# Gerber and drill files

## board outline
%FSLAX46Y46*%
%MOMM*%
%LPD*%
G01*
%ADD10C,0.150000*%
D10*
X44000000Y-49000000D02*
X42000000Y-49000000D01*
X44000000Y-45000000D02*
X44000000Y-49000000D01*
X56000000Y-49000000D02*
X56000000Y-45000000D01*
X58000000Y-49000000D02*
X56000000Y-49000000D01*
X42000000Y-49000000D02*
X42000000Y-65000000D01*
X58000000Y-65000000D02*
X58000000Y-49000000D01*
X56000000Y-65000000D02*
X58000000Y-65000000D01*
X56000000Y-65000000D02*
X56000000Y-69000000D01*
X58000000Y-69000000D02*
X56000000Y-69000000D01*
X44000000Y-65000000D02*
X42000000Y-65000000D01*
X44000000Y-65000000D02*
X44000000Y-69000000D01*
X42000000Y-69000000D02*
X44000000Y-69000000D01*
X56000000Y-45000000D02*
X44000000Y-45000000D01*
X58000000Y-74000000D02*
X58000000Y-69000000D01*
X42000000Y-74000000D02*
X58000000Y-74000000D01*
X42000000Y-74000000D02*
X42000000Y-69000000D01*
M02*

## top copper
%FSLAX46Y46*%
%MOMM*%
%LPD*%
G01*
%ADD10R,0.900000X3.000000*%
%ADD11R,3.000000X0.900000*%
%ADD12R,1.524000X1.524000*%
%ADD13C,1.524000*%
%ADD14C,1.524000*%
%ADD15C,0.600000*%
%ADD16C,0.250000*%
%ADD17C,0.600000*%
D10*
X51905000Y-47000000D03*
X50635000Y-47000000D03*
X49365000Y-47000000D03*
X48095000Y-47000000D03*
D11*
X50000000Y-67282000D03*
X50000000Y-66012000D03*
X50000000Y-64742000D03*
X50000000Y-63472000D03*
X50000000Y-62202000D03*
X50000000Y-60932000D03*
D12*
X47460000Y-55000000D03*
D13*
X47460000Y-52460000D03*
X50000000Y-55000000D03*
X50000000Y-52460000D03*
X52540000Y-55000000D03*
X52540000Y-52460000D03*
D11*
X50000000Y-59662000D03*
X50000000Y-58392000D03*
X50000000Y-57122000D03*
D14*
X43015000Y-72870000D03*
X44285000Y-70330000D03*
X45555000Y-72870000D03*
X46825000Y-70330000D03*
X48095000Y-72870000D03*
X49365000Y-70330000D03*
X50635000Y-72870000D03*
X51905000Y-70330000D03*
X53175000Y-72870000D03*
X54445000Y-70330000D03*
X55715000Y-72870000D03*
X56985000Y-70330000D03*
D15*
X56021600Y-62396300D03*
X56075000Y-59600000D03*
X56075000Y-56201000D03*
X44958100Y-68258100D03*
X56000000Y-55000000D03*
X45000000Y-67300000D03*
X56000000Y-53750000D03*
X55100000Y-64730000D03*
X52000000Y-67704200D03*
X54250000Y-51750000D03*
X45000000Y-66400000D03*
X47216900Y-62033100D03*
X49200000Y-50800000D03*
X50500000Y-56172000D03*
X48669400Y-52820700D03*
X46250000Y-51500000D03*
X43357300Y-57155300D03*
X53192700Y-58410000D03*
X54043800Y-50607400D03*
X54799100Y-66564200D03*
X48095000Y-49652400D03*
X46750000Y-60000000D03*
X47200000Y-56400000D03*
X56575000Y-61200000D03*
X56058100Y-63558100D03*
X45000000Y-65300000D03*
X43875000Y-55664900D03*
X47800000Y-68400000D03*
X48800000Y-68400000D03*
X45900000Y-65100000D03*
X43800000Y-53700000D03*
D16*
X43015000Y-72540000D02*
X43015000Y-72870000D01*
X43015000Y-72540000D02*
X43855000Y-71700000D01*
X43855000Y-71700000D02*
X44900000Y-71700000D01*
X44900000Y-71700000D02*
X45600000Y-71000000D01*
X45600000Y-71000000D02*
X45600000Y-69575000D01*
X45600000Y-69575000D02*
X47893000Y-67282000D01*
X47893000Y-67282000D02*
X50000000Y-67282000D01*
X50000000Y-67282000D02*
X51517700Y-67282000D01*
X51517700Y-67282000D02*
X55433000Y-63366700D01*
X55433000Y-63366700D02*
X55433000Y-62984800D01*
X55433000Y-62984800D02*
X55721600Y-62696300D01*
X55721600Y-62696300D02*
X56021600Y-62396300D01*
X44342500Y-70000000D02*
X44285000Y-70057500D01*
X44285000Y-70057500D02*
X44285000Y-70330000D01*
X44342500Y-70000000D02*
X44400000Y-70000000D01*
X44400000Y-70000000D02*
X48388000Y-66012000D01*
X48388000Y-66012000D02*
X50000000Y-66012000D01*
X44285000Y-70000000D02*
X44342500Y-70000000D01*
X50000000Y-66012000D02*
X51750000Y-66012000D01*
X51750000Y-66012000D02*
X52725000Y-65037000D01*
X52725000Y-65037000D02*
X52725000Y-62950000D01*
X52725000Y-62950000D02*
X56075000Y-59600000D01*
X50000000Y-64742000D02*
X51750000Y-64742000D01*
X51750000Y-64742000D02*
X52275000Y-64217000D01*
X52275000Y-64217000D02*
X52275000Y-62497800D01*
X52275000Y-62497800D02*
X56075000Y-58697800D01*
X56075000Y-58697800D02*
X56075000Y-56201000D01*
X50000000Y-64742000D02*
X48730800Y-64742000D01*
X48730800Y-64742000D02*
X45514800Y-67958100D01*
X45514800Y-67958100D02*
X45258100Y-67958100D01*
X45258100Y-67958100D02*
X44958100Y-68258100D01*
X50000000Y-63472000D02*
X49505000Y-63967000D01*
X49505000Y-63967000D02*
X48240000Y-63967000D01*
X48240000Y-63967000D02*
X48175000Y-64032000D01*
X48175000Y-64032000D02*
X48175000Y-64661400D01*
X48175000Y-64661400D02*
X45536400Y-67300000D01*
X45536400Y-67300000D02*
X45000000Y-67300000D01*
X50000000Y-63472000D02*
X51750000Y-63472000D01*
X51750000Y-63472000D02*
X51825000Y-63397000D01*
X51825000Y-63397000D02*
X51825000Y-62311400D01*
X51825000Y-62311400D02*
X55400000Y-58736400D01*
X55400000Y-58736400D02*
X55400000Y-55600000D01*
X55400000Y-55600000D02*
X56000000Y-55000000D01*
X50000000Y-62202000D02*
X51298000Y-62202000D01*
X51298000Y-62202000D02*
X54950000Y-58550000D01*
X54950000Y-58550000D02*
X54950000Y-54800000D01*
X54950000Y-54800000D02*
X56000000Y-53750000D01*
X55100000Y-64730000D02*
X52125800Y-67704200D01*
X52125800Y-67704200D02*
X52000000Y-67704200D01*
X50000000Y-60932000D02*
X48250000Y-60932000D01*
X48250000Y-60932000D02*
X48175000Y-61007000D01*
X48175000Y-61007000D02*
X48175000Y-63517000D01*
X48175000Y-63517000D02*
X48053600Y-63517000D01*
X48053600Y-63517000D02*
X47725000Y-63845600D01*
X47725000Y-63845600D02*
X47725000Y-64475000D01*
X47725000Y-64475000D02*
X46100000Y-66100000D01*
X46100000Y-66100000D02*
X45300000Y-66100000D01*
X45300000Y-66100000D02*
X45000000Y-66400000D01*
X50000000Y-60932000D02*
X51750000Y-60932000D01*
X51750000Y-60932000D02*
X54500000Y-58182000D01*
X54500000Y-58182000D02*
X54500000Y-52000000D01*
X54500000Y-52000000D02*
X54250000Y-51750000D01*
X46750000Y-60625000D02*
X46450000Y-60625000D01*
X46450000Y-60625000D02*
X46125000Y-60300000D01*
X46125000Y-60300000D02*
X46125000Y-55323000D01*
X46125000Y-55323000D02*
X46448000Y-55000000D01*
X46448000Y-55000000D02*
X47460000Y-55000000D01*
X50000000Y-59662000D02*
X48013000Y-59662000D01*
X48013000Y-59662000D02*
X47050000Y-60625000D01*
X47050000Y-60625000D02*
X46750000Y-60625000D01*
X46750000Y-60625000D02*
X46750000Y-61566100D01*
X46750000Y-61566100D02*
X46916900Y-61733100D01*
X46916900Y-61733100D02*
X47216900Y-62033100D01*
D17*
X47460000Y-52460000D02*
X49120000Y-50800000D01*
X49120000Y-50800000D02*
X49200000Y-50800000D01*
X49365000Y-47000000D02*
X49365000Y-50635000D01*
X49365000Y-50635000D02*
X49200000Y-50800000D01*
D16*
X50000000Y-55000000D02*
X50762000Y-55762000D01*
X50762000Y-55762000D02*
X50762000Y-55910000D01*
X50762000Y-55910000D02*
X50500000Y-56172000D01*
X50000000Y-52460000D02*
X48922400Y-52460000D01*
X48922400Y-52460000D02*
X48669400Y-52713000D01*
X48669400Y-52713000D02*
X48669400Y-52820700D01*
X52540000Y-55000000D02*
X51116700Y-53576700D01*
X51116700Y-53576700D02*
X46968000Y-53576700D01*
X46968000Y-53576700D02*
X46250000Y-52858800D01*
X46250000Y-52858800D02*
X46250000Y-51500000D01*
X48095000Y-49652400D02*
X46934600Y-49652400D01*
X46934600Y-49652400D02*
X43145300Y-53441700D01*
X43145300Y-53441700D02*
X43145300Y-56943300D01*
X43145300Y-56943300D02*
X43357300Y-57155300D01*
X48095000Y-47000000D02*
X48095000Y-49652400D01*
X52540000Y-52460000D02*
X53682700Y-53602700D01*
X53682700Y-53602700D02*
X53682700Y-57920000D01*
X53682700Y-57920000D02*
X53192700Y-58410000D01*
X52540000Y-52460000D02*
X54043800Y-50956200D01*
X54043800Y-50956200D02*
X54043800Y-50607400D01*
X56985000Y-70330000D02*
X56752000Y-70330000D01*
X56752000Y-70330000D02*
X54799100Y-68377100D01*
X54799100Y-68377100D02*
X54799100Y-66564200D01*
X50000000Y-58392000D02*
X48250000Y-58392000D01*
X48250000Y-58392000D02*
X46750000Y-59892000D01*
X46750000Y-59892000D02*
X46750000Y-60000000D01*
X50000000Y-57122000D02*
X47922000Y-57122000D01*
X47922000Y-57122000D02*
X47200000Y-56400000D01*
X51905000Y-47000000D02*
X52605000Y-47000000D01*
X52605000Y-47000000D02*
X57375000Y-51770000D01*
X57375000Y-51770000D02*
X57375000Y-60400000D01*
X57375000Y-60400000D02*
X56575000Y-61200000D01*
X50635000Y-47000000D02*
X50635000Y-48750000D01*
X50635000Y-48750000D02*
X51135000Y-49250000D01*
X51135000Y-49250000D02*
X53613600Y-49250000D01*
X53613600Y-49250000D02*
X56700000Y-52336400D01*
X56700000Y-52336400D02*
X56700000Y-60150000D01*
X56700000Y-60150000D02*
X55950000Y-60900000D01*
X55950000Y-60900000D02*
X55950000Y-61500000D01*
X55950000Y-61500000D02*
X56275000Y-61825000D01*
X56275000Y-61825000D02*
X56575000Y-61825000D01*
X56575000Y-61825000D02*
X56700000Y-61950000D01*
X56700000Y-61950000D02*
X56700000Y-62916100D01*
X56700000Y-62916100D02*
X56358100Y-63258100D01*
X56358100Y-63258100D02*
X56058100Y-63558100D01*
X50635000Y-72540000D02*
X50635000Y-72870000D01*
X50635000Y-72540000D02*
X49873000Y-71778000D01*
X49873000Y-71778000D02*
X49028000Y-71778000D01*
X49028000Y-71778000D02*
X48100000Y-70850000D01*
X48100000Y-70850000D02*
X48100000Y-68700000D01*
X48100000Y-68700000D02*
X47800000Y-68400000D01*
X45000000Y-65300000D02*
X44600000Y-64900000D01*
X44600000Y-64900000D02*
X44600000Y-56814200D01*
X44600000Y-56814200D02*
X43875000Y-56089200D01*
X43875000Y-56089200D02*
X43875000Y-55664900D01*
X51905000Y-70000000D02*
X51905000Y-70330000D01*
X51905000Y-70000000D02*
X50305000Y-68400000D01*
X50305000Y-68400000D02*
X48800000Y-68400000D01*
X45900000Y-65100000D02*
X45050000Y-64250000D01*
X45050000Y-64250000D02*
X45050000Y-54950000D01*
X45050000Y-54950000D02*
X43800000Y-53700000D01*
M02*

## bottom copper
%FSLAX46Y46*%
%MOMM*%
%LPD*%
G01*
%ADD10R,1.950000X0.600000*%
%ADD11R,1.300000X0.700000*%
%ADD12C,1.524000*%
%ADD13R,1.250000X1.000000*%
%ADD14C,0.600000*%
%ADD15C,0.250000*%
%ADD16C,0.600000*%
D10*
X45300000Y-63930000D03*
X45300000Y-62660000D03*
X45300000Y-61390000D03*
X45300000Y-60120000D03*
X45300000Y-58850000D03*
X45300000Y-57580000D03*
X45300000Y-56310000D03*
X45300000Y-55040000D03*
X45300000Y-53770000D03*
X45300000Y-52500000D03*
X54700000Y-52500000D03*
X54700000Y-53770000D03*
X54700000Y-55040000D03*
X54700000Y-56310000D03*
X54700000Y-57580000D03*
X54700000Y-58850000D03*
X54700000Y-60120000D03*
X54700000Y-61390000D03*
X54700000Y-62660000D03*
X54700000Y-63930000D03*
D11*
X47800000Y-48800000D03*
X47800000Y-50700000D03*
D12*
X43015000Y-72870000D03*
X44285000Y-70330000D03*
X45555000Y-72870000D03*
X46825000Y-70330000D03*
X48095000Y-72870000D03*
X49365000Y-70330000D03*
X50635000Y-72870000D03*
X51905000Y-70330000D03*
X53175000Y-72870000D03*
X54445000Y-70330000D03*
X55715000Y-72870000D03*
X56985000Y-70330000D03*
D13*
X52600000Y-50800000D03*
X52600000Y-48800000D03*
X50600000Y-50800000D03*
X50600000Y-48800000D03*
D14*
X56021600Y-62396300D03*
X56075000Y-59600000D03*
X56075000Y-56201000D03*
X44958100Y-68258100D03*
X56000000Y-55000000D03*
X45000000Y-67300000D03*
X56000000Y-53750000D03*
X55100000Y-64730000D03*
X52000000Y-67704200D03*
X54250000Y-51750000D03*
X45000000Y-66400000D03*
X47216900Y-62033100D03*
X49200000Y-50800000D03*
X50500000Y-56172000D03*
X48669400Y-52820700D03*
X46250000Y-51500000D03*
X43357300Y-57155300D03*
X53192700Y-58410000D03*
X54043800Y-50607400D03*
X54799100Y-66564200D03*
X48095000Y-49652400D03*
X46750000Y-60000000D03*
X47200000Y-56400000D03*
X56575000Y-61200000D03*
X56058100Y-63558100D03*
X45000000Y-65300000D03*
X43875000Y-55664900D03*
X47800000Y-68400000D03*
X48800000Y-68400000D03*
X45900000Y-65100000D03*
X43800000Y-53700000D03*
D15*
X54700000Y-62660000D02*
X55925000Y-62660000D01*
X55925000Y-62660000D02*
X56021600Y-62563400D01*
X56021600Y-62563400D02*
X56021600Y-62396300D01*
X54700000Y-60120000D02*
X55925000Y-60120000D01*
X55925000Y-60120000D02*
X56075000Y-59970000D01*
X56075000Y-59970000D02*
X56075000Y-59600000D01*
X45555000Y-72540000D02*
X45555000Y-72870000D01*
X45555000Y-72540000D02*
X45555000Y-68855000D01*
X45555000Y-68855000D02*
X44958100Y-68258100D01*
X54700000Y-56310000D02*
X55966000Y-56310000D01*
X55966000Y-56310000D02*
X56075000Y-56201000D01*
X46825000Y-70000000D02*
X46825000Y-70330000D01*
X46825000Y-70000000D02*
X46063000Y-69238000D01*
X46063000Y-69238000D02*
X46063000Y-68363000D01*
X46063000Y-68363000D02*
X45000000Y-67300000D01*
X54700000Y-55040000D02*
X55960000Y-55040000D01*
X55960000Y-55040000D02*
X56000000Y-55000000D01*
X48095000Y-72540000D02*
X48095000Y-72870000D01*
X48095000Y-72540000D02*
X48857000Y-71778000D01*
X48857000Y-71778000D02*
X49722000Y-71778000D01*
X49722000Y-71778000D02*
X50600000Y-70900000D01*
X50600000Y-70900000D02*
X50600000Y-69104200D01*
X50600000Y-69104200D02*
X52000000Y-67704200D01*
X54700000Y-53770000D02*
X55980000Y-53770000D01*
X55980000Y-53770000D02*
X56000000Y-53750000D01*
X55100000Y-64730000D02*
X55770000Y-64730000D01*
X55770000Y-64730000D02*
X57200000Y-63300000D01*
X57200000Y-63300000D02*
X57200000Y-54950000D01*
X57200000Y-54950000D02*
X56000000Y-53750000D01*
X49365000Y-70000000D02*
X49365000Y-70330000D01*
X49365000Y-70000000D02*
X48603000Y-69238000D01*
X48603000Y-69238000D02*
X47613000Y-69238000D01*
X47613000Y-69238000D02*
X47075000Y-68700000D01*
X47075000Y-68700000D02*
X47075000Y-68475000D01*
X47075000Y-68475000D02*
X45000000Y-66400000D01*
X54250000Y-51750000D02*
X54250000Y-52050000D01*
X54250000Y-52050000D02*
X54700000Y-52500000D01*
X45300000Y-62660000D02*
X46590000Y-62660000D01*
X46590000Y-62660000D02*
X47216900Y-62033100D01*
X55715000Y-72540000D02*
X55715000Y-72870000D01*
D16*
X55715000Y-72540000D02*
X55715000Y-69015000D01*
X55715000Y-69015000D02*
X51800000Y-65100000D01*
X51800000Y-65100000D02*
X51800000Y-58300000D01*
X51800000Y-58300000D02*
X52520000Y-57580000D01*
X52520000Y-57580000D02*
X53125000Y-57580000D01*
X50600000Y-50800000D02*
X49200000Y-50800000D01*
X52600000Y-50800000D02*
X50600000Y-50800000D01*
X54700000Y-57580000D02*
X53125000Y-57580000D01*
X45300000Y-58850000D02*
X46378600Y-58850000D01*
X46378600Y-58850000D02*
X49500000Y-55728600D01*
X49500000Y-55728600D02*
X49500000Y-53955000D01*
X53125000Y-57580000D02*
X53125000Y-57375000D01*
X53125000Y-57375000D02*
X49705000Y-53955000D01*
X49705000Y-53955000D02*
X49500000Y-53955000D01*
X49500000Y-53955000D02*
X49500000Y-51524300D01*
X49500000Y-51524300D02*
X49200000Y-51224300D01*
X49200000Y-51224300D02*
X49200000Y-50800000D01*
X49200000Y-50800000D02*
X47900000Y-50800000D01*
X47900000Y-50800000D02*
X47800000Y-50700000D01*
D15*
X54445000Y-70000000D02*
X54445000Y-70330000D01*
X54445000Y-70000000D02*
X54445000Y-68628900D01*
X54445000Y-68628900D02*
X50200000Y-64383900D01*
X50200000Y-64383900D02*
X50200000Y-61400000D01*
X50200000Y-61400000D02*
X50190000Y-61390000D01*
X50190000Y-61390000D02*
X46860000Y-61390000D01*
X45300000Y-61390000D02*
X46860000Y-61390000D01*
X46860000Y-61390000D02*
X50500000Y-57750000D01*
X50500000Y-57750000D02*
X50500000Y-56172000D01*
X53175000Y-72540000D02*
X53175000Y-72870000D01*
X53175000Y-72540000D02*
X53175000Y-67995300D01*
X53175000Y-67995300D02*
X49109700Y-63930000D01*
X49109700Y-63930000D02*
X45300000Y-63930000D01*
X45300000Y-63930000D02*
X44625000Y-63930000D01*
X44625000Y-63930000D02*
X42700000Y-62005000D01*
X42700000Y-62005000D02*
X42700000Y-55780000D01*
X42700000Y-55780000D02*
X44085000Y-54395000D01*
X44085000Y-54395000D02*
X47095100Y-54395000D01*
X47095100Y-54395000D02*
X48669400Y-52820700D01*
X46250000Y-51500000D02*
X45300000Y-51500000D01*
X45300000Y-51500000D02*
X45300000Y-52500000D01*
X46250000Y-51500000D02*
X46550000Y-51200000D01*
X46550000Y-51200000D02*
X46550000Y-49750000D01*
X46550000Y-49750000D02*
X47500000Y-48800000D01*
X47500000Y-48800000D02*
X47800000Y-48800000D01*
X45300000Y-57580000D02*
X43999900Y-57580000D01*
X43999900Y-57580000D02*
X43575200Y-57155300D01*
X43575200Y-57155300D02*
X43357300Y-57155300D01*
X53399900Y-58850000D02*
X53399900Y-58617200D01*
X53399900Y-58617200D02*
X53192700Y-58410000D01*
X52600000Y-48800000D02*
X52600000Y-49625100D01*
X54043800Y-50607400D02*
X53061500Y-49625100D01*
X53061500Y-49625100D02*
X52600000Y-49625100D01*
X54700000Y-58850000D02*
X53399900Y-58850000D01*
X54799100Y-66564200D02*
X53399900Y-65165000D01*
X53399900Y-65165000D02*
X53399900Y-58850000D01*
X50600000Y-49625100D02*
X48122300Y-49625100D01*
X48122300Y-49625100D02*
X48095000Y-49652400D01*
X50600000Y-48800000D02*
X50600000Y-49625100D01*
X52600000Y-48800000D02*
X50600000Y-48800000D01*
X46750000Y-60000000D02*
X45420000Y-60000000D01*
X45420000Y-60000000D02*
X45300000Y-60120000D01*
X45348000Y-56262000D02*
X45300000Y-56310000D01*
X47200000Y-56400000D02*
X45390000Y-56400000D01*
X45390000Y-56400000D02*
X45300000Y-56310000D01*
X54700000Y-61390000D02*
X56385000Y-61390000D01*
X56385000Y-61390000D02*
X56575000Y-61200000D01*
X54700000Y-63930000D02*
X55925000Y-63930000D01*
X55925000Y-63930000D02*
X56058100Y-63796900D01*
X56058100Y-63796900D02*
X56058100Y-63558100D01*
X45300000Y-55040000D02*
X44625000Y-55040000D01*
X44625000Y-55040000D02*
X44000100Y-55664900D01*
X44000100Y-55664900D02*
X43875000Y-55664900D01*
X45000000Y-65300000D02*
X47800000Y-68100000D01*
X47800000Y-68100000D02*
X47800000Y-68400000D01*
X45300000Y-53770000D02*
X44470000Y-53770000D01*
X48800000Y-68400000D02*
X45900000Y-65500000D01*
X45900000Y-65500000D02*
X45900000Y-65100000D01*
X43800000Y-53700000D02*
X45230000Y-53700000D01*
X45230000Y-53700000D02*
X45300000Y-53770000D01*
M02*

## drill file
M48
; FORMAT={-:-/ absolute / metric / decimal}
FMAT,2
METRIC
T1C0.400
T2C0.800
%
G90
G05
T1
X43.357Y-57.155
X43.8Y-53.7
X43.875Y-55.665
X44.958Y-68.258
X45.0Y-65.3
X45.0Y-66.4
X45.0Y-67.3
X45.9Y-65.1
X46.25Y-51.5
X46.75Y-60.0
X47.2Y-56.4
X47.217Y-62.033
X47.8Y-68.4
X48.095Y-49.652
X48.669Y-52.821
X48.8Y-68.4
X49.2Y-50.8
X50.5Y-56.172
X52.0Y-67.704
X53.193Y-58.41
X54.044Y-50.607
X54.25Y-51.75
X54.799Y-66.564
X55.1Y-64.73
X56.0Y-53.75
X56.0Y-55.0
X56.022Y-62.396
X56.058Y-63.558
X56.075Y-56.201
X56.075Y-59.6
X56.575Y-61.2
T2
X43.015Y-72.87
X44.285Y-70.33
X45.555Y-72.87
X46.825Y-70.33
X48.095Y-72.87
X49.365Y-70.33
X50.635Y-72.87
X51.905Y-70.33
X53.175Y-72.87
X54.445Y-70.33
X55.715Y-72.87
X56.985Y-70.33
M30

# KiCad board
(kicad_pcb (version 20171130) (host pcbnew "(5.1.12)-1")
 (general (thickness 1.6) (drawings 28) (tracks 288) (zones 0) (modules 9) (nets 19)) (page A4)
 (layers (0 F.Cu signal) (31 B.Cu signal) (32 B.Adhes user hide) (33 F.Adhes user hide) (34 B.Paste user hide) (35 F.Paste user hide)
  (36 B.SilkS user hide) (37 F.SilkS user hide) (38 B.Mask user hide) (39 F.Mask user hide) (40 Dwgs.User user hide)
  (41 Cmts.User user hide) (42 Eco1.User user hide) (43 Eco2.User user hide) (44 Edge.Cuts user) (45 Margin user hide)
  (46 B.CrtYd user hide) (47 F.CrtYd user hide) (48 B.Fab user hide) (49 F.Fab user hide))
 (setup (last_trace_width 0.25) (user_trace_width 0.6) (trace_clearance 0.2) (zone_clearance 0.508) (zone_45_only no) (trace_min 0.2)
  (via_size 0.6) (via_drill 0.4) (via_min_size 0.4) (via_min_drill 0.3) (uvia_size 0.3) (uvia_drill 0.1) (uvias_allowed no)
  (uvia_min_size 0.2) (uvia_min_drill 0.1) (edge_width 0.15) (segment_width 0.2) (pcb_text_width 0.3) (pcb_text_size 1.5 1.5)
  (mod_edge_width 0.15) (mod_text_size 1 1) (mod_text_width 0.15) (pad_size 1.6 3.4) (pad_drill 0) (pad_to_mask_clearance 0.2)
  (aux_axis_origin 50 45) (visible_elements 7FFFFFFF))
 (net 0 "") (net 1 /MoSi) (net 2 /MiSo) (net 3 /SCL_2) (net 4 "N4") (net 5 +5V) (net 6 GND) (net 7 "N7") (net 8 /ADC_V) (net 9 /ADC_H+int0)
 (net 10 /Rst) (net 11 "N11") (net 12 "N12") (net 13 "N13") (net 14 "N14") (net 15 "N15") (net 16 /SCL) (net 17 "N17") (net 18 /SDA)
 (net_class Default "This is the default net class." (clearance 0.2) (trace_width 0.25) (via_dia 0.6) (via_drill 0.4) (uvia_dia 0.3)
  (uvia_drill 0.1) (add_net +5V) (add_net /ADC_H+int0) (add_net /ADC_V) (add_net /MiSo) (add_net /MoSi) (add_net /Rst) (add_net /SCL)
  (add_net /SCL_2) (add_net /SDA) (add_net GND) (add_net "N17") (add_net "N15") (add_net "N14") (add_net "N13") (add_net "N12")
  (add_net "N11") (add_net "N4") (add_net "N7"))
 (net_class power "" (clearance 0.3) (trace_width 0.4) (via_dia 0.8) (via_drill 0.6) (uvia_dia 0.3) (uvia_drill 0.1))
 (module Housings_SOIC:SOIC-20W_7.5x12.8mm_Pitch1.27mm (layer B.Cu) (at 50 58.215)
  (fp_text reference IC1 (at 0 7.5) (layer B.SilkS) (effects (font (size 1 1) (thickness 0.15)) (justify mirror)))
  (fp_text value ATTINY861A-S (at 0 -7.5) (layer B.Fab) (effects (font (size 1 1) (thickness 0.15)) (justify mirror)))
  (pad 1 smd rect (at -4.7 5.715) (size 1.95 0.6) (layers B.Cu B.Paste B.Mask) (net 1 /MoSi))
  (pad 2 smd rect (at -4.7 4.445) (size 1.95 0.6) (layers B.Cu B.Paste B.Mask) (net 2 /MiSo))
  (pad 3 smd rect (at -4.7 3.175) (size 1.95 0.6) (layers B.Cu B.Paste B.Mask) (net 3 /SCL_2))
  (pad 4 smd rect (at -4.7 1.905) (size 1.95 0.6) (layers B.Cu B.Paste B.Mask) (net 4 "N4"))
  (pad 5 smd rect (at -4.7 0.635) (size 1.95 0.6) (layers B.Cu B.Paste B.Mask) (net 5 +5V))
  (pad 6 smd rect (at -4.7 -0.635) (size 1.95 0.6) (layers B.Cu B.Paste B.Mask) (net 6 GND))
  (pad 7 smd rect (at -4.7 -1.905) (size 1.95 0.6) (layers B.Cu B.Paste B.Mask) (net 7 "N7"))
  (pad 8 smd rect (at -4.7 -3.175) (size 1.95 0.6) (layers B.Cu B.Paste B.Mask) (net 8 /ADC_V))
  (pad 9 smd rect (at -4.7 -4.445) (size 1.95 0.6) (layers B.Cu B.Paste B.Mask) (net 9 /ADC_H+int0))
  (pad 10 smd rect (at -4.7 -5.715) (size 1.95 0.6) (layers B.Cu B.Paste B.Mask) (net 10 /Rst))
  (pad 11 smd rect (at 4.7 -5.715) (size 1.95 0.6) (layers B.Cu B.Paste B.Mask) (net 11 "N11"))
  (pad 12 smd rect (at 4.7 -4.445) (size 1.95 0.6) (layers B.Cu B.Paste B.Mask) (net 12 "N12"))
  (pad 13 smd rect (at 4.7 -3.175) (size 1.95 0.6) (layers B.Cu B.Paste B.Mask) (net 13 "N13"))
  (pad 14 smd rect (at 4.7 -1.905) (size 1.95 0.6) (layers B.Cu B.Paste B.Mask) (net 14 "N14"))
  (pad 15 smd rect (at 4.7 -0.635) (size 1.95 0.6) (layers B.Cu B.Paste B.Mask) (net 5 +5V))
  (pad 16 smd rect (at 4.7 0.635) (size 1.95 0.6) (layers B.Cu B.Paste B.Mask) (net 6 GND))
  (pad 17 smd rect (at 4.7 1.905) (size 1.95 0.6) (layers B.Cu B.Paste B.Mask) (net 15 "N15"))
  (pad 18 smd rect (at 4.7 3.175) (size 1.95 0.6) (layers B.Cu B.Paste B.Mask) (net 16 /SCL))
  (pad 19 smd rect (at 4.7 4.445) (size 1.95 0.6) (layers B.Cu B.Paste B.Mask) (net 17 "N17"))
  (pad 20 smd rect (at 4.7 5.715) (size 1.95 0.6) (layers B.Cu B.Paste B.Mask) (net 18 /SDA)))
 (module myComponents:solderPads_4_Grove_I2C (layer F.Cu) (at 50 47 180)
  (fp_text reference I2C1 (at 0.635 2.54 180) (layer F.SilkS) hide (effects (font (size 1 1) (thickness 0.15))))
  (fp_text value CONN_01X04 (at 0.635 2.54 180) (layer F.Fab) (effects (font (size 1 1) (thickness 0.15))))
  (pad 1 smd rect (at -1.905 0 180) (size 0.9 3) (layers F.Cu F.Paste F.Mask) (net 16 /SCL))
  (pad 2 smd rect (at -0.635 0 180) (size 0.9 3) (layers F.Cu F.Paste F.Mask) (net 18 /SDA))
  (pad 3 smd rect (at 0.635 0 180) (size 0.9 3) (layers F.Cu F.Paste F.Mask) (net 5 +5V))
  (pad 4 smd rect (at 1.905 0 180) (size 0.9 3) (layers F.Cu F.Paste F.Mask) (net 6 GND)))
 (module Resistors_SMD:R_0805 (layer B.Cu) (at 47.8 49.75 270)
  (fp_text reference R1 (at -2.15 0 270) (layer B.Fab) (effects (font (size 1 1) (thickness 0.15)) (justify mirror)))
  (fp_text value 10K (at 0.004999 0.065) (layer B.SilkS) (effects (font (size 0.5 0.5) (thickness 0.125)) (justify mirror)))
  (pad 1 smd rect (at -0.95 0 270) (size 0.7 1.3) (layers B.Cu B.Paste B.Mask) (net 10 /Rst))
  (pad 2 smd rect (at 0.95 0 270) (size 0.7 1.3) (layers B.Cu B.Paste B.Mask) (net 5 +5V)))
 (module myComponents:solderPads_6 (layer F.Cu) (at 50 64.107 90)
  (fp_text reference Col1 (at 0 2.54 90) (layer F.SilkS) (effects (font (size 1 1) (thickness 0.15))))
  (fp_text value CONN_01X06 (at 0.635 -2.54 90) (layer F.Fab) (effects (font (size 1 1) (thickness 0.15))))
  (pad 1 smd rect (at -3.175 0 90) (size 0.9 3) (layers F.Cu F.Paste F.Mask) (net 17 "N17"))
  (pad 2 smd rect (at -1.905 0 90) (size 0.9 3) (layers F.Cu F.Paste F.Mask) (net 15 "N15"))
  (pad 3 smd rect (at -0.635 0 90) (size 0.9 3) (layers F.Cu F.Paste F.Mask) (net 14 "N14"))
  (pad 4 smd rect (at 0.635 0 90) (size 0.9 3) (layers F.Cu F.Paste F.Mask) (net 13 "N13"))
  (pad 5 smd rect (at 1.905 0 90) (size 0.9 3) (layers F.Cu F.Paste F.Mask) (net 12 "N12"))
  (pad 6 smd rect (at 3.175 0 90) (size 0.9 3) (layers F.Cu F.Paste F.Mask) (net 11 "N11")))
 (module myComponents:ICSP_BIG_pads (layer F.Cu) (at 50 53.73 90)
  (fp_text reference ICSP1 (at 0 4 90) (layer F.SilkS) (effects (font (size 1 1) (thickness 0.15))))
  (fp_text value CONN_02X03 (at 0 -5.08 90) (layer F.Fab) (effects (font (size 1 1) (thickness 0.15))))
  (pad 1 smd rect (at -1.27 -2.54 90) (size 1.524 1.524) (layers F.Cu F.Paste F.Mask) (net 2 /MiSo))
  (pad 2 smd circle (at 1.27 -2.54 90) (size 1.524 1.524) (layers F.Cu F.Paste F.Mask) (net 5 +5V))
  (pad 3 smd circle (at -1.27 0 90) (size 1.524 1.524) (layers F.Cu F.Paste F.Mask) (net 3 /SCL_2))
  (pad 4 smd circle (at 1.27 0 90) (size 1.524 1.524) (layers F.Cu F.Paste F.Mask) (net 1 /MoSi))
  (pad 5 smd circle (at -1.27 2.54 90) (size 1.524 1.524) (layers F.Cu F.Paste F.Mask) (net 10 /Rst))
  (pad 6 smd circle (at 1.27 2.54 90) (size 1.524 1.524) (layers F.Cu F.Paste F.Mask) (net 6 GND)))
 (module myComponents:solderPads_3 (layer F.Cu) (at 50 58.392 90)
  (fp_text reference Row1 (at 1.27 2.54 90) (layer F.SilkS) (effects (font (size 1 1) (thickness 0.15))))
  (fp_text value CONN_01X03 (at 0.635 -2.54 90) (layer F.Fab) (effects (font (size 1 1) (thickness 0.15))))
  (pad 1 smd rect (at -1.27 0 90) (size 0.9 3) (layers F.Cu F.Paste F.Mask) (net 2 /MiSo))
  (pad 2 smd rect (at 0 0 90) (size 0.9 3) (layers F.Cu F.Paste F.Mask) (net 4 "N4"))
  (pad 3 smd rect (at 1.27 0 90) (size 0.9 3) (layers F.Cu F.Paste F.Mask) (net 7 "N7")))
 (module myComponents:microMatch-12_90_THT (layer F.Cu) (at 50 71.6)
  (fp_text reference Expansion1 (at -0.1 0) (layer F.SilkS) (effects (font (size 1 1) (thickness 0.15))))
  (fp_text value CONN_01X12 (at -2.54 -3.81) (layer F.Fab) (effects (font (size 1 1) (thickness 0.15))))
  (pad 1 thru_hole circle (at -6.985 1.27) (size 1.524 1.524) (drill 0.8) (layers *.Cu *.Mask) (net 17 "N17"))
  (pad 2 thru_hole circle (at -5.715 -1.27) (size 1.524 1.524) (drill 0.8) (layers *.Cu *.Mask) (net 15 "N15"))
  (pad 3 thru_hole circle (at -4.445 1.27) (size 1.524 1.524) (drill 0.8) (layers *.Cu *.Mask) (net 14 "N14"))
  (pad 4 thru_hole circle (at -3.175 -1.27) (size 1.524 1.524) (drill 0.8) (layers *.Cu *.Mask) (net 13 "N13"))
  (pad 5 thru_hole circle (at -1.905 1.27) (size 1.524 1.524) (drill 0.8) (layers *.Cu *.Mask) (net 12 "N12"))
  (pad 6 thru_hole circle (at -0.635 -1.27) (size 1.524 1.524) (drill 0.8) (layers *.Cu *.Mask) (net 11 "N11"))
  (pad 7 thru_hole circle (at 0.635 1.27) (size 1.524 1.524) (drill 0.8) (layers *.Cu *.Mask) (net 8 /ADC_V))
  (pad 8 thru_hole circle (at 1.905 -1.27) (size 1.524 1.524) (drill 0.8) (layers *.Cu *.Mask) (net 9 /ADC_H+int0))
  (pad 9 thru_hole circle (at 3.175 1.27) (size 1.524 1.524) (drill 0.8) (layers *.Cu *.Mask) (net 1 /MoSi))
  (pad 10 thru_hole circle (at 4.445 -1.27) (size 1.524 1.524) (drill 0.8) (layers *.Cu *.Mask) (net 3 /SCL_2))
  (pad 11 thru_hole circle (at 5.715 1.27) (size 1.524 1.524) (drill 0.8) (layers *.Cu *.Mask) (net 5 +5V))
  (pad 12 thru_hole circle (at 6.985 -1.27) (size 1.524 1.524) (drill 0.8) (layers *.Cu *.Mask) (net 6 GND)))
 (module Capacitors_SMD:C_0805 (layer B.Cu) (at 52.6 49.8 90)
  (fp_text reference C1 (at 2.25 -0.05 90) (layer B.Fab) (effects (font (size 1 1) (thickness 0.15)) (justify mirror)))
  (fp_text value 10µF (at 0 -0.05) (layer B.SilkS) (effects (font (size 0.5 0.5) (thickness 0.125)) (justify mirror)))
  (pad 1 smd rect (at -1 0 90) (size 1 1.25) (layers B.Cu B.Paste B.Mask) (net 5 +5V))
  (pad 2 smd rect (at 1 0 90) (size 1 1.25) (layers B.Cu B.Paste B.Mask) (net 6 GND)))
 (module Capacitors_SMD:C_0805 (layer B.Cu) (at 50.6 49.8 90)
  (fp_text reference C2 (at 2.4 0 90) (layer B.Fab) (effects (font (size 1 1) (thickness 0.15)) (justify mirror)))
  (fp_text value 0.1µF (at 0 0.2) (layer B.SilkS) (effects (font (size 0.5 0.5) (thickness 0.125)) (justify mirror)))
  (pad 1 smd rect (at -1 0 90) (size 1 1.25) (layers B.Cu B.Paste B.Mask) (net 5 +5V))
  (pad 2 smd rect (at 1 0 90) (size 1 1.25) (layers B.Cu B.Paste B.Mask) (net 6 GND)))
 (gr_line (start 44 49) (end 42 49) (layer Edge.Cuts) (width 0.15))
 (gr_line (start 44 45) (end 44 49) (layer Edge.Cuts) (width 0.15))
 (gr_line (start 56 49) (end 56 45) (layer Edge.Cuts) (width 0.15))
 (gr_line (start 58 49) (end 56 49) (layer Edge.Cuts) (width 0.15))
 (gr_line (start 42 49) (end 42 65) (layer Edge.Cuts) (width 0.15))
 (gr_line (start 58 65) (end 58 49) (layer Edge.Cuts) (width 0.15))
 (gr_line (start 56 65) (end 58 65) (layer Edge.Cuts) (width 0.15))
 (gr_line (start 56 65) (end 56 69) (layer Edge.Cuts) (width 0.15))
 (gr_line (start 58 69) (end 56 69) (layer Edge.Cuts) (width 0.15))
 (gr_line (start 44 65) (end 42 65) (layer Edge.Cuts) (width 0.15))
 (gr_line (start 44 65) (end 44 69) (layer Edge.Cuts) (width 0.15))
 (gr_line (start 42 69) (end 44 69) (layer Edge.Cuts) (width 0.15))
 (gr_line (start 56 45) (end 44 45) (layer Edge.Cuts) (width 0.15))
 (gr_line (start 58 74) (end 58 69) (layer Edge.Cuts) (width 0.15))
 (gr_line (start 42 74) (end 58 74) (layer Edge.Cuts) (width 0.15))
 (gr_line (start 42 74) (end 42 69) (layer Edge.Cuts) (width 0.15))
 (segment (start 43.015 72.54) (end 43.015 72.87) (width 0.25) (layer F.Cu) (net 17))
 (segment (start 43.015 72.54) (end 43.855 71.7) (width 0.25) (layer F.Cu) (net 17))
 (segment (start 43.855 71.7) (end 44.9 71.7) (width 0.25) (layer F.Cu) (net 17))
 (segment (start 44.9 71.7) (end 45.6 71) (width 0.25) (layer F.Cu) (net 17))
 (segment (start 45.6 71) (end 45.6 69.575) (width 0.25) (layer F.Cu) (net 17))
 (segment (start 45.6 69.575) (end 47.893 67.282) (width 0.25) (layer F.Cu) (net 17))
 (segment (start 47.893 67.282) (end 50 67.282) (width 0.25) (layer F.Cu) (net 17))
 (segment (start 54.7 62.66) (end 55.925 62.66) (width 0.25) (layer B.Cu) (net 17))
 (segment (start 55.925 62.66) (end 56.0216 62.5634) (width 0.25) (layer B.Cu) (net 17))
 (segment (start 56.0216 62.5634) (end 56.0216 62.3963) (width 0.25) (layer B.Cu) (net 17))
 (segment (start 50 67.282) (end 51.5177 67.282) (width 0.25) (layer F.Cu) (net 17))
 (segment (start 51.5177 67.282) (end 55.433 63.3667) (width 0.25) (layer F.Cu) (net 17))
 (segment (start 55.433 63.3667) (end 55.433 62.9848) (width 0.25) (layer F.Cu) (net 17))
 (segment (start 55.433 62.9848) (end 55.7216 62.6963) (width 0.25) (layer F.Cu) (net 17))
 (segment (start 55.7216 62.6963) (end 56.0216 62.3963) (width 0.25) (layer F.Cu) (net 17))
 (via (at 56.0216 62.3963) (size 0.6) (layers F.Cu B.Cu) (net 17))
 (segment (start 44.3425 70) (end 44.285 70.0575) (width 0.25) (layer F.Cu) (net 15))
 (segment (start 44.285 70.0575) (end 44.285 70.33) (width 0.25) (layer F.Cu) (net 15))
 (segment (start 44.3425 70) (end 44.4 70) (width 0.25) (layer F.Cu) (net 15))
 (segment (start 44.4 70) (end 48.388 66.012) (width 0.25) (layer F.Cu) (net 15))
 (segment (start 48.388 66.012) (end 50 66.012) (width 0.25) (layer F.Cu) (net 15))
 (segment (start 44.285 70) (end 44.3425 70) (width 0.25) (layer F.Cu) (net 15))
 (segment (start 50 66.012) (end 51.75 66.012) (width 0.25) (layer F.Cu) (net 15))
 (segment (start 51.75 66.012) (end 52.725 65.037) (width 0.25) (layer F.Cu) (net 15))
 (segment (start 52.725 65.037) (end 52.725 62.95) (width 0.25) (layer F.Cu) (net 15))
 (segment (start 52.725 62.95) (end 56.075 59.6) (width 0.25) (layer F.Cu) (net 15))
 (segment (start 54.7 60.12) (end 55.925 60.12) (width 0.25) (layer B.Cu) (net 15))
 (segment (start 55.925 60.12) (end 56.075 59.97) (width 0.25) (layer B.Cu) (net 15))
 (segment (start 56.075 59.97) (end 56.075 59.6) (width 0.25) (layer B.Cu) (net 15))
 (via (at 56.075 59.6) (size 0.6) (layers F.Cu B.Cu) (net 15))
 (segment (start 45.555 72.54) (end 45.555 72.87) (width 0.25) (layer B.Cu) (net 14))
 (segment (start 45.555 72.54) (end 45.555 68.855) (width 0.25) (layer B.Cu) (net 14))
 (segment (start 45.555 68.855) (end 44.9581 68.2581) (width 0.25) (layer B.Cu) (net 14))
 (segment (start 50 64.742) (end 51.75 64.742) (width 0.25) (layer F.Cu) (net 14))
 (segment (start 51.75 64.742) (end 52.275 64.217) (width 0.25) (layer F.Cu) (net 14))
 (segment (start 52.275 64.217) (end 52.275 62.4978) (width 0.25) (layer F.Cu) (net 14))
 (segment (start 52.275 62.4978) (end 56.075 58.6978) (width 0.25) (layer F.Cu) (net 14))
 (segment (start 56.075 58.6978) (end 56.075 56.201) (width 0.25) (layer F.Cu) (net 14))
 (segment (start 54.7 56.31) (end 55.966 56.31) (width 0.25) (layer B.Cu) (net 14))
 (segment (start 55.966 56.31) (end 56.075 56.201) (width 0.25) (layer B.Cu) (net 14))
 (segment (start 50 64.742) (end 48.7308 64.742) (width 0.25) (layer F.Cu) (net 14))
 (segment (start 48.7308 64.742) (end 45.5148 67.9581) (width 0.25) (layer F.Cu) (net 14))
 (segment (start 45.5148 67.9581) (end 45.2581 67.9581) (width 0.25) (layer F.Cu) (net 14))
 (segment (start 45.2581 67.9581) (end 44.9581 68.2581) (width 0.25) (layer F.Cu) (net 14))
 (via (at 56.075 56.201) (size 0.6) (layers F.Cu B.Cu) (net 14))
 (via (at 44.9581 68.2581) (size 0.6) (layers F.Cu B.Cu) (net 14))
 (segment (start 46.825 70) (end 46.825 70.33) (width 0.25) (layer B.Cu) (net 13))
 (segment (start 46.825 70) (end 46.063 69.238) (width 0.25) (layer B.Cu) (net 13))
 (segment (start 46.063 69.238) (end 46.063 68.363) (width 0.25) (layer B.Cu) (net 13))
 (segment (start 46.063 68.363) (end 45 67.3) (width 0.25) (layer B.Cu) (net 13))
 (segment (start 54.7 55.04) (end 55.96 55.04) (width 0.25) (layer B.Cu) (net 13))
 (segment (start 55.96 55.04) (end 56 55) (width 0.25) (layer B.Cu) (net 13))
 (segment (start 50 63.472) (end 49.505 63.967) (width 0.25) (layer F.Cu) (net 13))
 (segment (start 49.505 63.967) (end 48.24 63.967) (width 0.25) (layer F.Cu) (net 13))
 (segment (start 48.24 63.967) (end 48.175 64.032) (width 0.25) (layer F.Cu) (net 13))
 (segment (start 48.175 64.032) (end 48.175 64.6614) (width 0.25) (layer F.Cu) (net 13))
 (segment (start 48.175 64.6614) (end 45.5364 67.3) (width 0.25) (layer F.Cu) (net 13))
 (segment (start 45.5364 67.3) (end 45 67.3) (width 0.25) (layer F.Cu) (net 13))
 (segment (start 50 63.472) (end 51.75 63.472) (width 0.25) (layer F.Cu) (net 13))
 (segment (start 51.75 63.472) (end 51.825 63.397) (width 0.25) (layer F.Cu) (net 13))
 (segment (start 51.825 63.397) (end 51.825 62.3114) (width 0.25) (layer F.Cu) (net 13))
 (segment (start 51.825 62.3114) (end 55.4 58.7364) (width 0.25) (layer F.Cu) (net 13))
 (segment (start 55.4 58.7364) (end 55.4 55.6) (width 0.25) (layer F.Cu) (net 13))
 (segment (start 55.4 55.6) (end 56 55) (width 0.25) (layer F.Cu) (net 13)) (via (at 56 55) (size 0.6) (layers F.Cu B.Cu) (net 13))
 (via (at 45 67.3) (size 0.6) (layers F.Cu B.Cu) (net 13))
 (segment (start 48.095 72.54) (end 48.095 72.87) (width 0.25) (layer B.Cu) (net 12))
 (segment (start 48.095 72.54) (end 48.857 71.778) (width 0.25) (layer B.Cu) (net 12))
 (segment (start 48.857 71.778) (end 49.722 71.778) (width 0.25) (layer B.Cu) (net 12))
 (segment (start 49.722 71.778) (end 50.6 70.9) (width 0.25) (layer B.Cu) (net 12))
 (segment (start 50.6 70.9) (end 50.6 69.1042) (width 0.25) (layer B.Cu) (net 12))
 (segment (start 50.6 69.1042) (end 52 67.7042) (width 0.25) (layer B.Cu) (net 12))
 (segment (start 54.7 53.77) (end 55.98 53.77) (width 0.25) (layer B.Cu) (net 12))
 (segment (start 55.98 53.77) (end 56 53.75) (width 0.25) (layer B.Cu) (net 12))
 (segment (start 55.1 64.73) (end 55.77 64.73) (width 0.25) (layer B.Cu) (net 12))
 (segment (start 55.77 64.73) (end 57.2 63.3) (width 0.25) (layer B.Cu) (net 12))
 (segment (start 57.2 63.3) (end 57.2 54.95) (width 0.25) (layer B.Cu) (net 12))
 (segment (start 57.2 54.95) (end 56 53.75) (width 0.25) (layer B.Cu) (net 12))
 (segment (start 50 62.202) (end 51.298 62.202) (width 0.25) (layer F.Cu) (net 12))
 (segment (start 51.298 62.202) (end 54.95 58.55) (width 0.25) (layer F.Cu) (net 12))
 (segment (start 54.95 58.55) (end 54.95 54.8) (width 0.25) (layer F.Cu) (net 12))
 (segment (start 54.95 54.8) (end 56 53.75) (width 0.25) (layer F.Cu) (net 12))
 (segment (start 55.1 64.73) (end 52.1258 67.7042) (width 0.25) (layer F.Cu) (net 12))
 (segment (start 52.1258 67.7042) (end 52 67.7042) (width 0.25) (layer F.Cu) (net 12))
 (via (at 56 53.75) (size 0.6) (layers F.Cu B.Cu) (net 12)) (via (at 55.1 64.73) (size 0.6) (layers F.Cu B.Cu) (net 12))
 (via (at 52 67.7042) (size 0.6) (layers F.Cu B.Cu) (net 12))
 (segment (start 49.365 70) (end 49.365 70.33) (width 0.25) (layer B.Cu) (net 11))
 (segment (start 49.365 70) (end 48.603 69.238) (width 0.25) (layer B.Cu) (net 11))
 (segment (start 48.603 69.238) (end 47.613 69.238) (width 0.25) (layer B.Cu) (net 11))
 (segment (start 47.613 69.238) (end 47.075 68.7) (width 0.25) (layer B.Cu) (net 11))
 (segment (start 47.075 68.7) (end 47.075 68.475) (width 0.25) (layer B.Cu) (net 11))
 (segment (start 47.075 68.475) (end 45 66.4) (width 0.25) (layer B.Cu) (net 11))
 (segment (start 54.25 51.75) (end 54.25 52.05) (width 0.25) (layer B.Cu) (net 11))
 (segment (start 54.25 52.05) (end 54.7 52.5) (width 0.25) (layer B.Cu) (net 11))
 (segment (start 50 60.932) (end 48.25 60.932) (width 0.25) (layer F.Cu) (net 11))
 (segment (start 48.25 60.932) (end 48.175 61.007) (width 0.25) (layer F.Cu) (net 11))
 (segment (start 48.175 61.007) (end 48.175 63.517) (width 0.25) (layer F.Cu) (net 11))
 (segment (start 48.175 63.517) (end 48.0536 63.517) (width 0.25) (layer F.Cu) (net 11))
 (segment (start 48.0536 63.517) (end 47.725 63.8456) (width 0.25) (layer F.Cu) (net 11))
 (segment (start 47.725 63.8456) (end 47.725 64.475) (width 0.25) (layer F.Cu) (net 11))
 (segment (start 47.725 64.475) (end 46.1 66.1) (width 0.25) (layer F.Cu) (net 11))
 (segment (start 46.1 66.1) (end 45.3 66.1) (width 0.25) (layer F.Cu) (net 11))
 (segment (start 45.3 66.1) (end 45 66.4) (width 0.25) (layer F.Cu) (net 11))
 (segment (start 50 60.932) (end 51.75 60.932) (width 0.25) (layer F.Cu) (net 11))
 (segment (start 51.75 60.932) (end 54.5 58.182) (width 0.25) (layer F.Cu) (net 11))
 (segment (start 54.5 58.182) (end 54.5 52) (width 0.25) (layer F.Cu) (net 11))
 (segment (start 54.5 52) (end 54.25 51.75) (width 0.25) (layer F.Cu) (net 11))
 (via (at 54.25 51.75) (size 0.6) (layers F.Cu B.Cu) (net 11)) (via (at 45 66.4) (size 0.6) (layers F.Cu B.Cu) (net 11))
 (segment (start 46.75 60.625) (end 46.45 60.625) (width 0.25) (layer F.Cu) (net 2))
 (segment (start 46.45 60.625) (end 46.125 60.3) (width 0.25) (layer F.Cu) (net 2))
 (segment (start 46.125 60.3) (end 46.125 55.323) (width 0.25) (layer F.Cu) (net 2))
 (segment (start 46.125 55.323) (end 46.448 55) (width 0.25) (layer F.Cu) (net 2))
 (segment (start 46.448 55) (end 47.46 55) (width 0.25) (layer F.Cu) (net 2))
 (segment (start 50 59.662) (end 48.013 59.662) (width 0.25) (layer F.Cu) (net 2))
 (segment (start 48.013 59.662) (end 47.05 60.625) (width 0.25) (layer F.Cu) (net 2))
 (segment (start 47.05 60.625) (end 46.75 60.625) (width 0.25) (layer F.Cu) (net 2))
 (segment (start 45.3 62.66) (end 46.59 62.66) (width 0.25) (layer B.Cu) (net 2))
 (segment (start 46.59 62.66) (end 47.2169 62.0331) (width 0.25) (layer B.Cu) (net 2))
 (segment (start 46.75 60.625) (end 46.75 61.5661) (width 0.25) (layer F.Cu) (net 2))
 (segment (start 46.75 61.5661) (end 46.9169 61.7331) (width 0.25) (layer F.Cu) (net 2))
 (segment (start 46.9169 61.7331) (end 47.2169 62.0331) (width 0.25) (layer F.Cu) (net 2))
 (via (at 47.2169 62.0331) (size 0.6) (layers F.Cu B.Cu) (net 2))
 (segment (start 55.715 72.54) (end 55.715 72.87) (width 0.25) (layer B.Cu) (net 5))
 (segment (start 55.715 72.54) (end 55.715 69.015) (width 0.6) (layer B.Cu) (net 5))
 (segment (start 55.715 69.015) (end 51.8 65.1) (width 0.6) (layer B.Cu) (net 5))
 (segment (start 51.8 65.1) (end 51.8 58.3) (width 0.6) (layer B.Cu) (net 5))
 (segment (start 51.8 58.3) (end 52.52 57.58) (width 0.6) (layer B.Cu) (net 5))
 (segment (start 52.52 57.58) (end 53.125 57.58) (width 0.6) (layer B.Cu) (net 5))
 (segment (start 50.6 50.8) (end 49.2 50.8) (width 0.6) (layer B.Cu) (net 5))
 (segment (start 52.6 50.8) (end 50.6 50.8) (width 0.6) (layer B.Cu) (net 5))
 (segment (start 54.7 57.58) (end 53.125 57.58) (width 0.6) (layer B.Cu) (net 5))
 (segment (start 45.3 58.85) (end 46.3786 58.85) (width 0.6) (layer B.Cu) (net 5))
 (segment (start 46.3786 58.85) (end 49.5 55.7286) (width 0.6) (layer B.Cu) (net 5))
 (segment (start 49.5 55.7286) (end 49.5 53.955) (width 0.6) (layer B.Cu) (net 5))
 (segment (start 53.125 57.58) (end 53.125 57.375) (width 0.6) (layer B.Cu) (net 5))
 (segment (start 53.125 57.375) (end 49.705 53.955) (width 0.6) (layer B.Cu) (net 5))
 (segment (start 49.705 53.955) (end 49.5 53.955) (width 0.6) (layer B.Cu) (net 5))
 (segment (start 49.5 53.955) (end 49.5 51.5243) (width 0.6) (layer B.Cu) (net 5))
 (segment (start 49.5 51.5243) (end 49.2 51.2243) (width 0.6) (layer B.Cu) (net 5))
 (segment (start 49.2 51.2243) (end 49.2 50.8) (width 0.6) (layer B.Cu) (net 5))
 (segment (start 47.46 52.46) (end 49.12 50.8) (width 0.6) (layer F.Cu) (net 5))
 (segment (start 49.12 50.8) (end 49.2 50.8) (width 0.6) (layer F.Cu) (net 5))
 (segment (start 49.365 47) (end 49.365 50.635) (width 0.6) (layer F.Cu) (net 5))
 (segment (start 49.365 50.635) (end 49.2 50.8) (width 0.6) (layer F.Cu) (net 5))
 (segment (start 49.2 50.8) (end 47.9 50.8) (width 0.6) (layer B.Cu) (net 5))
 (segment (start 47.9 50.8) (end 47.8 50.7) (width 0.6) (layer B.Cu) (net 5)) (via (at 49.2 50.8) (size 0.6) (layers F.Cu B.Cu) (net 5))
 (segment (start 54.445 70) (end 54.445 70.33) (width 0.25) (layer B.Cu) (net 3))
 (segment (start 54.445 70) (end 54.445 68.6289) (width 0.25) (layer B.Cu) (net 3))
 (segment (start 54.445 68.6289) (end 50.2 64.3839) (width 0.25) (layer B.Cu) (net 3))
 (segment (start 50.2 64.3839) (end 50.2 61.4) (width 0.25) (layer B.Cu) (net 3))
 (segment (start 50.2 61.4) (end 50.19 61.39) (width 0.25) (layer B.Cu) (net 3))
 (segment (start 50.19 61.39) (end 46.86 61.39) (width 0.25) (layer B.Cu) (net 3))
 (segment (start 45.3 61.39) (end 46.86 61.39) (width 0.25) (layer B.Cu) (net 3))
 (segment (start 50 55) (end 50.762 55.762) (width 0.25) (layer F.Cu) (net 3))
 (segment (start 50.762 55.762) (end 50.762 55.91) (width 0.25) (layer F.Cu) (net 3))
 (segment (start 50.762 55.91) (end 50.5 56.172) (width 0.25) (layer F.Cu) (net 3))
 (segment (start 46.86 61.39) (end 50.5 57.75) (width 0.25) (layer B.Cu) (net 3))
 (segment (start 50.5 57.75) (end 50.5 56.172) (width 0.25) (layer B.Cu) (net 3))
 (via (at 50.5 56.172) (size 0.6) (layers F.Cu B.Cu) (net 3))
 (segment (start 53.175 72.54) (end 53.175 72.87) (width 0.25) (layer B.Cu) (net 1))
 (segment (start 53.175 72.54) (end 53.175 67.9953) (width 0.25) (layer B.Cu) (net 1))
 (segment (start 53.175 67.9953) (end 49.1097 63.93) (width 0.25) (layer B.Cu) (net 1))
 (segment (start 49.1097 63.93) (end 45.3 63.93) (width 0.25) (layer B.Cu) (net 1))
 (segment (start 45.3 63.93) (end 44.625 63.93) (width 0.25) (layer B.Cu) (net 1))
 (segment (start 44.625 63.93) (end 42.7 62.005) (width 0.25) (layer B.Cu) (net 1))
 (segment (start 42.7 62.005) (end 42.7 55.78) (width 0.25) (layer B.Cu) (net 1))
 (segment (start 42.7 55.78) (end 44.085 54.395) (width 0.25) (layer B.Cu) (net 1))
 (segment (start 44.085 54.395) (end 47.0951 54.395) (width 0.25) (layer B.Cu) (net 1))
 (segment (start 47.0951 54.395) (end 48.6694 52.8207) (width 0.25) (layer B.Cu) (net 1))
 (segment (start 50 52.46) (end 48.9224 52.46) (width 0.25) (layer F.Cu) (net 1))
 (segment (start 48.9224 52.46) (end 48.6694 52.713) (width 0.25) (layer F.Cu) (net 1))
 (segment (start 48.6694 52.713) (end 48.6694 52.8207) (width 0.25) (layer F.Cu) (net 1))
 (via (at 48.6694 52.8207) (size 0.6) (layers F.Cu B.Cu) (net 1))
 (segment (start 46.25 51.5) (end 45.3 51.5) (width 0.25) (layer B.Cu) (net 10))
 (segment (start 45.3 51.5) (end 45.3 52.5) (width 0.25) (layer B.Cu) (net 10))
 (segment (start 52.54 55) (end 51.1167 53.5767) (width 0.25) (layer F.Cu) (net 10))
 (segment (start 51.1167 53.5767) (end 46.968 53.5767) (width 0.25) (layer F.Cu) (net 10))
 (segment (start 46.968 53.5767) (end 46.25 52.8588) (width 0.25) (layer F.Cu) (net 10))
 (segment (start 46.25 52.8588) (end 46.25 51.5) (width 0.25) (layer F.Cu) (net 10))
 (segment (start 46.25 51.5) (end 46.55 51.2) (width 0.25) (layer B.Cu) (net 10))
 (segment (start 46.55 51.2) (end 46.55 49.75) (width 0.25) (layer B.Cu) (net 10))
 (segment (start 46.55 49.75) (end 47.5 48.8) (width 0.25) (layer B.Cu) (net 10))
 (segment (start 47.5 48.8) (end 47.8 48.8) (width 0.25) (layer B.Cu) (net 10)) (via (at 46.25 51.5) (size 0.6) (layers F.Cu B.Cu) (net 10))
 (segment (start 48.095 49.6524) (end 46.9346 49.6524) (width 0.25) (layer F.Cu) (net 6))
 (segment (start 46.9346 49.6524) (end 43.1453 53.4417) (width 0.25) (layer F.Cu) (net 6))
 (segment (start 43.1453 53.4417) (end 43.1453 56.9433) (width 0.25) (layer F.Cu) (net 6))
 (segment (start 43.1453 56.9433) (end 43.3573 57.1553) (width 0.25) (layer F.Cu) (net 6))
 (segment (start 48.095 47) (end 48.095 49.6524) (width 0.25) (layer F.Cu) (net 6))
 (segment (start 45.3 57.58) (end 43.9999 57.58) (width 0.25) (layer B.Cu) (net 6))
 (segment (start 43.9999 57.58) (end 43.5752 57.1553) (width 0.25) (layer B.Cu) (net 6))
 (segment (start 43.5752 57.1553) (end 43.3573 57.1553) (width 0.25) (layer B.Cu) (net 6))
 (segment (start 52.54 52.46) (end 53.6827 53.6027) (width 0.25) (layer F.Cu) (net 6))
 (segment (start 53.6827 53.6027) (end 53.6827 57.92) (width 0.25) (layer F.Cu) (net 6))
 (segment (start 53.6827 57.92) (end 53.1927 58.41) (width 0.25) (layer F.Cu) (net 6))
 (segment (start 53.3999 58.85) (end 53.3999 58.6172) (width 0.25) (layer B.Cu) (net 6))
 (segment (start 53.3999 58.6172) (end 53.1927 58.41) (width 0.25) (layer B.Cu) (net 6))
 (segment (start 52.54 52.46) (end 54.0438 50.9562) (width 0.25) (layer F.Cu) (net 6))
 (segment (start 54.0438 50.9562) (end 54.0438 50.6074) (width 0.25) (layer F.Cu) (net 6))
 (segment (start 52.6 48.8) (end 52.6 49.6251) (width 0.25) (layer B.Cu) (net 6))
 (segment (start 54.0438 50.6074) (end 53.0615 49.6251) (width 0.25) (layer B.Cu) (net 6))
 (segment (start 53.0615 49.6251) (end 52.6 49.6251) (width 0.25) (layer B.Cu) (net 6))
 (segment (start 54.7 58.85) (end 53.3999 58.85) (width 0.25) (layer B.Cu) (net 6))
 (segment (start 54.7991 66.5642) (end 53.3999 65.165) (width 0.25) (layer B.Cu) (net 6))
 (segment (start 53.3999 65.165) (end 53.3999 58.85) (width 0.25) (layer B.Cu) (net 6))
 (segment (start 56.985 70.33) (end 56.752 70.33) (width 0.25) (layer F.Cu) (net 6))
 (segment (start 56.752 70.33) (end 54.7991 68.3771) (width 0.25) (layer F.Cu) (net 6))
 (segment (start 54.7991 68.3771) (end 54.7991 66.5642) (width 0.25) (layer F.Cu) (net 6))
 (segment (start 50.6 49.6251) (end 48.1223 49.6251) (width 0.25) (layer B.Cu) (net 6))
 (segment (start 48.1223 49.6251) (end 48.095 49.6524) (width 0.25) (layer B.Cu) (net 6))
 (segment (start 50.6 48.8) (end 50.6 49.6251) (width 0.25) (layer B.Cu) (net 6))
 (segment (start 52.6 48.8) (end 50.6 48.8) (width 0.25) (layer B.Cu) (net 6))
 (via (at 43.3573 57.1553) (size 0.6) (layers F.Cu B.Cu) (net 6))
 (via (at 53.1927 58.41) (size 0.6) (layers F.Cu B.Cu) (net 6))
 (via (at 54.0438 50.6074) (size 0.6) (layers F.Cu B.Cu) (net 6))
 (via (at 54.7991 66.5642) (size 0.6) (layers F.Cu B.Cu) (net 6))
 (via (at 48.095 49.6524) (size 0.6) (layers F.Cu B.Cu) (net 6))
 (segment (start 50 58.392) (end 48.25 58.392) (width 0.25) (layer F.Cu) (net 4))
 (segment (start 48.25 58.392) (end 46.75 59.892) (width 0.25) (layer F.Cu) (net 4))
 (segment (start 46.75 59.892) (end 46.75 60) (width 0.25) (layer F.Cu) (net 4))
 (segment (start 46.75 60) (end 45.42 60) (width 0.25) (layer B.Cu) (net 4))
 (segment (start 45.42 60) (end 45.3 60.12) (width 0.25) (layer B.Cu) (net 4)) (via (at 46.75 60) (size 0.6) (layers F.Cu B.Cu) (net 4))
 (segment (start 45.348 56.262) (end 45.3 56.31) (width 0.25) (layer B.Cu) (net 7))
 (segment (start 50 57.122) (end 47.922 57.122) (width 0.25) (layer F.Cu) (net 7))
 (segment (start 47.922 57.122) (end 47.2 56.4) (width 0.25) (layer F.Cu) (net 7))
 (segment (start 47.2 56.4) (end 45.39 56.4) (width 0.25) (layer B.Cu) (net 7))
 (segment (start 45.39 56.4) (end 45.3 56.31) (width 0.25) (layer B.Cu) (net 7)) (via (at 47.2 56.4) (size 0.6) (layers F.Cu B.Cu) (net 7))
 (segment (start 54.7 61.39) (end 56.385 61.39) (width 0.25) (layer B.Cu) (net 16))
 (segment (start 56.385 61.39) (end 56.575 61.2) (width 0.25) (layer B.Cu) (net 16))
 (segment (start 51.905 47) (end 52.605 47) (width 0.25) (layer F.Cu) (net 16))
 (segment (start 52.605 47) (end 57.375 51.77) (width 0.25) (layer F.Cu) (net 16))
 (segment (start 57.375 51.77) (end 57.375 60.4) (width 0.25) (layer F.Cu) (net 16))
 (segment (start 57.375 60.4) (end 56.575 61.2) (width 0.25) (layer F.Cu) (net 16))
 (via (at 56.575 61.2) (size 0.6) (layers F.Cu B.Cu) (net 16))
 (segment (start 50.635 47) (end 50.635 48.75) (width 0.25) (layer F.Cu) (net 18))
 (segment (start 50.635 48.75) (end 51.135 49.25) (width 0.25) (layer F.Cu) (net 18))
 (segment (start 51.135 49.25) (end 53.6136 49.25) (width 0.25) (layer F.Cu) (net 18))
 (segment (start 53.6136 49.25) (end 56.7 52.3364) (width 0.25) (layer F.Cu) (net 18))
 (segment (start 56.7 52.3364) (end 56.7 60.15) (width 0.25) (layer F.Cu) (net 18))
 (segment (start 56.7 60.15) (end 55.95 60.9) (width 0.25) (layer F.Cu) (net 18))
 (segment (start 55.95 60.9) (end 55.95 61.5) (width 0.25) (layer F.Cu) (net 18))
 (segment (start 55.95 61.5) (end 56.275 61.825) (width 0.25) (layer F.Cu) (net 18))
 (segment (start 56.275 61.825) (end 56.575 61.825) (width 0.25) (layer F.Cu) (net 18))
 (segment (start 56.575 61.825) (end 56.7 61.95) (width 0.25) (layer F.Cu) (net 18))
 (segment (start 56.7 61.95) (end 56.7 62.9161) (width 0.25) (layer F.Cu) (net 18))
 (segment (start 56.7 62.9161) (end 56.3581 63.2581) (width 0.25) (layer F.Cu) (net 18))
 (segment (start 56.3581 63.2581) (end 56.0581 63.5581) (width 0.25) (layer F.Cu) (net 18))
 (segment (start 54.7 63.93) (end 55.925 63.93) (width 0.25) (layer B.Cu) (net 18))
 (segment (start 55.925 63.93) (end 56.0581 63.7969) (width 0.25) (layer B.Cu) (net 18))
 (segment (start 56.0581 63.7969) (end 56.0581 63.5581) (width 0.25) (layer B.Cu) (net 18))
 (via (at 56.0581 63.5581) (size 0.6) (layers F.Cu B.Cu) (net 18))
 (segment (start 50.635 72.54) (end 50.635 72.87) (width 0.25) (layer F.Cu) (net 8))
 (segment (start 50.635 72.54) (end 49.873 71.778) (width 0.25) (layer F.Cu) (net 8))
 (segment (start 49.873 71.778) (end 49.028 71.778) (width 0.25) (layer F.Cu) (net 8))
 (segment (start 49.028 71.778) (end 48.1 70.85) (width 0.25) (layer F.Cu) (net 8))
 (segment (start 48.1 70.85) (end 48.1 68.7) (width 0.25) (layer F.Cu) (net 8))
 (segment (start 48.1 68.7) (end 47.8 68.4) (width 0.25) (layer F.Cu) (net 8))
 (segment (start 45.3 55.04) (end 44.625 55.04) (width 0.25) (layer B.Cu) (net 8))
 (segment (start 44.625 55.04) (end 44.0001 55.6649) (width 0.25) (layer B.Cu) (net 8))
 (segment (start 44.0001 55.6649) (end 43.875 55.6649) (width 0.25) (layer B.Cu) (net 8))
 (segment (start 45 65.3) (end 44.6 64.9) (width 0.25) (layer F.Cu) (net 8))
 (segment (start 44.6 64.9) (end 44.6 56.8142) (width 0.25) (layer F.Cu) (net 8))
 (segment (start 44.6 56.8142) (end 43.875 56.0892) (width 0.25) (layer F.Cu) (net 8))
 (segment (start 43.875 56.0892) (end 43.875 55.6649) (width 0.25) (layer F.Cu) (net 8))
 (segment (start 45 65.3) (end 47.8 68.1) (width 0.25) (layer B.Cu) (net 8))
 (segment (start 47.8 68.1) (end 47.8 68.4) (width 0.25) (layer B.Cu) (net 8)) (via (at 45 65.3) (size 0.6) (layers F.Cu B.Cu) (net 8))
 (via (at 43.875 55.6649) (size 0.6) (layers F.Cu B.Cu) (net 8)) (via (at 47.8 68.4) (size 0.6) (layers F.Cu B.Cu) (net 8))
 (segment (start 51.905 70) (end 51.905 70.33) (width 0.25) (layer F.Cu) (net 9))
 (segment (start 51.905 70) (end 50.305 68.4) (width 0.25) (layer F.Cu) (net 9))
 (segment (start 50.305 68.4) (end 48.8 68.4) (width 0.25) (layer F.Cu) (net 9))
 (segment (start 45.3 53.77) (end 44.47 53.77) (width 0.25) (layer B.Cu) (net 9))
 (segment (start 48.8 68.4) (end 45.9 65.5) (width 0.25) (layer B.Cu) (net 9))
 (segment (start 45.9 65.5) (end 45.9 65.1) (width 0.25) (layer B.Cu) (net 9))
 (segment (start 43.8 53.7) (end 45.23 53.7) (width 0.25) (layer B.Cu) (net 9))
 (segment (start 45.23 53.7) (end 45.3 53.77) (width 0.25) (layer B.Cu) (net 9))
 (segment (start 45.9 65.1) (end 45.05 64.25) (width 0.25) (layer F.Cu) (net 9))
 (segment (start 45.05 64.25) (end 45.05 54.95) (width 0.25) (layer F.Cu) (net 9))
 (segment (start 45.05 54.95) (end 43.8 53.7) (width 0.25) (layer F.Cu) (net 9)) (via (at 48.8 68.4) (size 0.6) (layers F.Cu B.Cu) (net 9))
 (via (at 45.9 65.1) (size 0.6) (layers F.Cu B.Cu) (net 9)) (via (at 43.8 53.7) (size 0.6) (layers F.Cu B.Cu) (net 9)))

